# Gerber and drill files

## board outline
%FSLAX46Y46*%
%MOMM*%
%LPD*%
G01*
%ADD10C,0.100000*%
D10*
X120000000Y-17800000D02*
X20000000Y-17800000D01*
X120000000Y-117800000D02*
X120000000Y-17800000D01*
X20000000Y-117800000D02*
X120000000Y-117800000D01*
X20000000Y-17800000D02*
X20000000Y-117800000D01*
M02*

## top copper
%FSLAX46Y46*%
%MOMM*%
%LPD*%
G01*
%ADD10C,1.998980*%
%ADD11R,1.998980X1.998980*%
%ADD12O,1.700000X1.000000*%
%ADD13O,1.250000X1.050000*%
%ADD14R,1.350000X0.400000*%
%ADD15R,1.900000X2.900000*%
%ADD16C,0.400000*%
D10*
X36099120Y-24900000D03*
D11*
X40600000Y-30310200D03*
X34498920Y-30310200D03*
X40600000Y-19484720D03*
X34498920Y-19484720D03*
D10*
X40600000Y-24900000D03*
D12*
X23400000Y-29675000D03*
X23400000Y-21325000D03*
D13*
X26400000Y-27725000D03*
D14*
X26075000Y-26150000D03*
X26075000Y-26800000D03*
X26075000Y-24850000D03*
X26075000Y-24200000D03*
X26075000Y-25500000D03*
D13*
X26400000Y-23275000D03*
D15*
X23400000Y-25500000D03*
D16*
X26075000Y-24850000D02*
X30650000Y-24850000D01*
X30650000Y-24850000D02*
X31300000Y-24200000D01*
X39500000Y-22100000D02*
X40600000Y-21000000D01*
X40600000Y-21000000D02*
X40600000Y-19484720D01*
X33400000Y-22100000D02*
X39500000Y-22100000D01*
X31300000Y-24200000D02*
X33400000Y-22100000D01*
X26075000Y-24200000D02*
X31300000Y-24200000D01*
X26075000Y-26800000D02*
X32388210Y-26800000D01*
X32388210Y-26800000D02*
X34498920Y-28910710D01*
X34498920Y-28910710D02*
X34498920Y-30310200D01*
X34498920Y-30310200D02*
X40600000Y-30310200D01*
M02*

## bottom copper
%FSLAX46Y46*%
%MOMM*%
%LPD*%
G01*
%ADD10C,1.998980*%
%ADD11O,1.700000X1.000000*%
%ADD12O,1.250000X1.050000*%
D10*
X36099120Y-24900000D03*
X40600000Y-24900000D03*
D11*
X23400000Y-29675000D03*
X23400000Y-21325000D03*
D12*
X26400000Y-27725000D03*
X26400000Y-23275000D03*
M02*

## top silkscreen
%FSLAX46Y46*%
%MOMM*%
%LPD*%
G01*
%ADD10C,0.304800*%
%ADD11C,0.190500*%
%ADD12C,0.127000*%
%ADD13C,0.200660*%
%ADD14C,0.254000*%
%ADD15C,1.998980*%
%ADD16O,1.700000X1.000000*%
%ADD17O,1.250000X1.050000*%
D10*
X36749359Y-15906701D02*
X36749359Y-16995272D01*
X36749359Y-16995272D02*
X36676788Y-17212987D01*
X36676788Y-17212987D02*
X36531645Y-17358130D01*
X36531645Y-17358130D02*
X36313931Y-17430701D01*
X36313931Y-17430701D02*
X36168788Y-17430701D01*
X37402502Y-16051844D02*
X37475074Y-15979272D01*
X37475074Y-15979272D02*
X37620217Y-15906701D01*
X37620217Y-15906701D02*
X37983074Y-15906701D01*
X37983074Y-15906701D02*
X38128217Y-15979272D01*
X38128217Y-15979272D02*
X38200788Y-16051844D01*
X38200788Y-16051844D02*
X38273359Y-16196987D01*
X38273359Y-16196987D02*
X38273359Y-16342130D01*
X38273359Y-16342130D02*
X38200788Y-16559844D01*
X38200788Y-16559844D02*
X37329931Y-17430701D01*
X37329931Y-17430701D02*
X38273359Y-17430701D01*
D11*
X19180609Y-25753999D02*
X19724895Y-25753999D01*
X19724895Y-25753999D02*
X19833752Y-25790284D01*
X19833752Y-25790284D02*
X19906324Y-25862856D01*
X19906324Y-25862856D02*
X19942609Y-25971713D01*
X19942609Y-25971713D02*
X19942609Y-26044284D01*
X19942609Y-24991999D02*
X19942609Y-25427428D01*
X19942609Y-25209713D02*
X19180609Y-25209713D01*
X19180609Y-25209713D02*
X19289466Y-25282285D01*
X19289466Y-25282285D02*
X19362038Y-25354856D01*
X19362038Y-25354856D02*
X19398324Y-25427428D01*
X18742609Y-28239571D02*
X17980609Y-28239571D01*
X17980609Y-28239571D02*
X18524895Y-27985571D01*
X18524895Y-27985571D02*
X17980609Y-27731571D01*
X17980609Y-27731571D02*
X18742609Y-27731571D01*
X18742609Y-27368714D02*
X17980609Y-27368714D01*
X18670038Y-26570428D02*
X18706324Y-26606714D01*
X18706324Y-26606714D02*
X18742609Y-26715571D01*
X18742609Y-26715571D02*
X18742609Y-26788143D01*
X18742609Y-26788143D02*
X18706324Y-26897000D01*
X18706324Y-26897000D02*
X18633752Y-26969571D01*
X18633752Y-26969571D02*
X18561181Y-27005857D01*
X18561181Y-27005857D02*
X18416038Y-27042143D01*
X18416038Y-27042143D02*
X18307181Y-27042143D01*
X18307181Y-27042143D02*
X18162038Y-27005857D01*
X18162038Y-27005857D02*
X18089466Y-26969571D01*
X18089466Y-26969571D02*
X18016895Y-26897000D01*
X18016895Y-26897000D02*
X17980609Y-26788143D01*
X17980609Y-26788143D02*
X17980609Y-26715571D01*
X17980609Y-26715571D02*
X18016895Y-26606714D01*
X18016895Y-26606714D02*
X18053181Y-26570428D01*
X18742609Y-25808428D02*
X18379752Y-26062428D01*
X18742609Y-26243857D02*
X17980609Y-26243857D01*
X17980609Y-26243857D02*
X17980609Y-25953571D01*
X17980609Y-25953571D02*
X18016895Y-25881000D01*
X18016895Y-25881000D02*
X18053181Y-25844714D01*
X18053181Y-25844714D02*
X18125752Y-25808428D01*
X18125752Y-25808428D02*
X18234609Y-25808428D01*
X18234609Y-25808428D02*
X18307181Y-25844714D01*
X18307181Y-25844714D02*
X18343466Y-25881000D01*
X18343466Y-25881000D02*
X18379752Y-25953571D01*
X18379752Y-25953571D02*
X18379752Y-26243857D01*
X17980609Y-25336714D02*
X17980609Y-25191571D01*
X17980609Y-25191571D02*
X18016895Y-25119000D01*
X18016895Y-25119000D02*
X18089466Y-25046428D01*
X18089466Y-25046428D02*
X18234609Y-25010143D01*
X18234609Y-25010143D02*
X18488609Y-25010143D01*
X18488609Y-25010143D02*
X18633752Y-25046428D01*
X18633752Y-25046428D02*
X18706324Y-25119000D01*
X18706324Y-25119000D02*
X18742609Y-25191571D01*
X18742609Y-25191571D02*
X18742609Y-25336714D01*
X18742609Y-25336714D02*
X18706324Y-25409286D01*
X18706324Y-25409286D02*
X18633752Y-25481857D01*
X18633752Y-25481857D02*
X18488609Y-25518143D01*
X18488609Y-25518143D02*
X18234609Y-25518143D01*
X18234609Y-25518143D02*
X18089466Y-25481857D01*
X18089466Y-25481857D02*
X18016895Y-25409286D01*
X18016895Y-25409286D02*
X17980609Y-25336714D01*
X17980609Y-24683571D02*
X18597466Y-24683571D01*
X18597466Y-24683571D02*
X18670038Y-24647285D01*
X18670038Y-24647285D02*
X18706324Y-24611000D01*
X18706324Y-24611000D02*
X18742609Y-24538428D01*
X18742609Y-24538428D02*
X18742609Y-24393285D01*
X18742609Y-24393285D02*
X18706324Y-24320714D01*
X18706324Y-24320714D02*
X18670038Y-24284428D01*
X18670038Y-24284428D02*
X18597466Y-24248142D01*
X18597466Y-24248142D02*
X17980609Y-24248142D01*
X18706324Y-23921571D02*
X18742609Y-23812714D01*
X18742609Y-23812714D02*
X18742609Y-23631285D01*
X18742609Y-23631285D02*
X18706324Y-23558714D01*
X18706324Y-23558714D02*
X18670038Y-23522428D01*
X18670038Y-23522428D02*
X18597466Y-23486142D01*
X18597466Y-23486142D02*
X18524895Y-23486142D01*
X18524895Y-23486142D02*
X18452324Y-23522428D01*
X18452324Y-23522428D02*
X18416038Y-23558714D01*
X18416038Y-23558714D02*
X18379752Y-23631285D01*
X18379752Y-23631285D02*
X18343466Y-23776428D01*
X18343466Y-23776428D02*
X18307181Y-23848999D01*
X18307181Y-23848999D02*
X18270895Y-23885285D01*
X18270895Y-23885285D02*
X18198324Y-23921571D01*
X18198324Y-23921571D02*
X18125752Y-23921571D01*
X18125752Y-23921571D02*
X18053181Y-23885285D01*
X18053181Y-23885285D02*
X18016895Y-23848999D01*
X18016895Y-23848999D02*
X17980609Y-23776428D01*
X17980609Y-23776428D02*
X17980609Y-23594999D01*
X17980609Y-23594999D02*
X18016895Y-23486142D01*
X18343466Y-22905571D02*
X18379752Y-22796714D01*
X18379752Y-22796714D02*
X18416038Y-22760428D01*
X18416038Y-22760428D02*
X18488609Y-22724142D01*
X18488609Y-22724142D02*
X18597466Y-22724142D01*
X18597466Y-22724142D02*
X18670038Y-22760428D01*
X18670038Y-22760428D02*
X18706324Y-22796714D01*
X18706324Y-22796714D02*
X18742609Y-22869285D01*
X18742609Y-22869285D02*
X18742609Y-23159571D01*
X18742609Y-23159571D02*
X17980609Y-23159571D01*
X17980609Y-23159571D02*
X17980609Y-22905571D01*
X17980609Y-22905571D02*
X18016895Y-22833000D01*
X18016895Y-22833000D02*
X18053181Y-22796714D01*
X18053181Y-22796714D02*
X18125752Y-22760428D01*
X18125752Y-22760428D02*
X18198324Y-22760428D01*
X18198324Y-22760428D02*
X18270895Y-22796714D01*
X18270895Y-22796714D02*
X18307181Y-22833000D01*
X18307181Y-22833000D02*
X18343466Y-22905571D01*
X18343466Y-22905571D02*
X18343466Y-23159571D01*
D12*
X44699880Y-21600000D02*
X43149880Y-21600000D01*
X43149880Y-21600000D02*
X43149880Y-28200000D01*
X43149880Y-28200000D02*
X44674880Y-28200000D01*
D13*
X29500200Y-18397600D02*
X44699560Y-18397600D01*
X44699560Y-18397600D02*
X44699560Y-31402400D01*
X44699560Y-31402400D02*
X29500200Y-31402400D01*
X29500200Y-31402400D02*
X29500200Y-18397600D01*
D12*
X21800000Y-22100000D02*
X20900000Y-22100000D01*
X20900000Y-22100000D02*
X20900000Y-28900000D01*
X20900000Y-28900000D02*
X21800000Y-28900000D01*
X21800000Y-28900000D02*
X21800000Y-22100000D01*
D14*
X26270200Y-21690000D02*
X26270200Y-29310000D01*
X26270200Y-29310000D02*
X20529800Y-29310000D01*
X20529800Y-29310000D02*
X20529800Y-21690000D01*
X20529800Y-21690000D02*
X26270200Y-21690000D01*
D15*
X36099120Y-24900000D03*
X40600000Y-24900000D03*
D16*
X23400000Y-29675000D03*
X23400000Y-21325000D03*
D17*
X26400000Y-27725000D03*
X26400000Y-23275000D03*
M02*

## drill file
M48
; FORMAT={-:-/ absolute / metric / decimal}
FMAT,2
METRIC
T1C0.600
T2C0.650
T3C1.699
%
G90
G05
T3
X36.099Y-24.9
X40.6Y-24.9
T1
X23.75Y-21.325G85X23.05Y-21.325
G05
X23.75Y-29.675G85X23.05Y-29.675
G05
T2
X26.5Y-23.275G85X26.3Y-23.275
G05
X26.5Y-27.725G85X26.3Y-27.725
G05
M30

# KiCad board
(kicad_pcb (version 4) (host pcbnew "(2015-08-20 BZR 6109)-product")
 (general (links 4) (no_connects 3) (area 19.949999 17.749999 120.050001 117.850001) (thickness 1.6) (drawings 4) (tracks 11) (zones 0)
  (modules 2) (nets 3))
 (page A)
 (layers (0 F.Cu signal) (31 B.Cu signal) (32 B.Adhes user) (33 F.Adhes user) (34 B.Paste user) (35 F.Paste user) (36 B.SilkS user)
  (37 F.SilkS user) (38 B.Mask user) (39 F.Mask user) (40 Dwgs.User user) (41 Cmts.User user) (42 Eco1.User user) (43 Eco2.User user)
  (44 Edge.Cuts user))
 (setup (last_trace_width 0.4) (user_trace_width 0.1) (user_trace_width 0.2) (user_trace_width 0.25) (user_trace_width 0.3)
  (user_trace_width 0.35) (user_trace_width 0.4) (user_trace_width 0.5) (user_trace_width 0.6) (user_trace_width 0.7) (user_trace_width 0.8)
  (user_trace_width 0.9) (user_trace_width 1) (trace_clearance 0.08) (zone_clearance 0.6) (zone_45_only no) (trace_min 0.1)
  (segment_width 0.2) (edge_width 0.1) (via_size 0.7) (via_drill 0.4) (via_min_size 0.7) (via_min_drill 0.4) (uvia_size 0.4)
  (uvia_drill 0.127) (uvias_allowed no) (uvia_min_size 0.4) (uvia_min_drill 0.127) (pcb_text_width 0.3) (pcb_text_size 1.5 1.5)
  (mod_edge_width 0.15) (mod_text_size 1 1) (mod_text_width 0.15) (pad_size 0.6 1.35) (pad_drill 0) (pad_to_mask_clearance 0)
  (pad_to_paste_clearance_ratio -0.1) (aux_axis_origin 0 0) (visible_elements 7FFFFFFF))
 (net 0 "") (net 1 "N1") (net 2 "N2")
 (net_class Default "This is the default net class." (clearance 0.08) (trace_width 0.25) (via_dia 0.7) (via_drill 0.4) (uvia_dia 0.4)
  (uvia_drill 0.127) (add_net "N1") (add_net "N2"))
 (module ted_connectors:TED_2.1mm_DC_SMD (layer F.Cu) (at 37.09988 24.9)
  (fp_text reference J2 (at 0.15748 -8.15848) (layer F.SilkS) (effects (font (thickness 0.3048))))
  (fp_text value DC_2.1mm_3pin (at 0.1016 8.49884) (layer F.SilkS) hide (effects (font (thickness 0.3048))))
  (fp_line (start 7.6 -3.3) (end 6.05 -3.3) (layer F.SilkS) (width 0.127))
  (fp_line (start 6.05 -3.3) (end 6.05 3.3) (layer F.SilkS) (width 0.127))
  (fp_line (start 6.05 3.3) (end 7.575 3.3) (layer F.SilkS) (width 0.127))
  (fp_line (start -7.59968 -6.5024) (end 7.59968 -6.5024) (layer F.SilkS) (width 0.20066))
  (fp_line (start 7.59968 -6.5024) (end 7.59968 6.5024) (layer F.SilkS) (width 0.20066))
  (fp_line (start 7.59968 6.5024) (end -7.59968 6.5024) (layer F.SilkS) (width 0.20066))
  (fp_line (start -7.59968 6.5024) (end -7.59968 -6.5024) (layer F.SilkS) (width 0.20066))
  (pad "" np_thru_hole circle (at -1.00076 0) (size 1.99898 1.99898) (drill 1.69926) (layers *.Cu *.Mask F.SilkS))
  (pad 1 smd rect (at 3.50012 5.4102) (size 1.99898 1.99898) (layers F.Cu F.Paste F.Mask) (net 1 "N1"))
  (pad 1 smd rect (at -2.60096 5.4102) (size 1.99898 1.99898) (layers F.Cu F.Paste F.Mask) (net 1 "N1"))
  (pad 2 smd rect (at 3.50012 -5.41528) (size 1.99898 1.99898) (layers F.Cu F.Paste F.Mask) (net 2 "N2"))
  (pad 3 smd rect (at -2.60096 -5.41528) (size 1.99898 1.99898) (layers F.Cu F.Paste F.Mask))
  (pad "" np_thru_hole circle (at 3.50012 0) (size 1.99898 1.99898) (drill 1.69926) (layers *.Cu *.Mask F.SilkS)))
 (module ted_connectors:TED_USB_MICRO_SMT (layer F.Cu) (at 23.4 25.5 270)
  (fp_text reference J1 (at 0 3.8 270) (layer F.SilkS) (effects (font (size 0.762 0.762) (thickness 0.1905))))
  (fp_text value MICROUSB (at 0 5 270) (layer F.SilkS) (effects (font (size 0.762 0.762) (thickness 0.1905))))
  (fp_line (start -3.4 1.6) (end -3.4 2.5) (layer F.SilkS) (width 0.127))
  (fp_line (start -3.4 2.5) (end 3.4 2.5) (layer F.SilkS) (width 0.127))
  (fp_line (start 3.4 2.5) (end 3.4 1.6) (layer F.SilkS) (width 0.127))
  (fp_line (start 3.4 1.6) (end -3.4 1.6) (layer F.SilkS) (width 0.127))
  (fp_line (start -3.81 -2.8702) (end 3.81 -2.8702) (layer F.SilkS) (width 0.254))
  (fp_line (start 3.81 -2.8702) (end 3.81 2.8702) (layer F.SilkS) (width 0.254))
  (fp_line (start 3.81 2.8702) (end -3.81 2.8702) (layer F.SilkS) (width 0.254))
  (fp_line (start -3.81 2.8702) (end -3.81 -2.8702) (layer F.SilkS) (width 0.254))
  (pad "" np_thru_hole oval (at 4.175 0 270) (size 1 1.7) (drill oval 0.6 1.3) (layers *.Cu *.Mask F.SilkS) (clearance 0.127))
  (pad "" np_thru_hole oval (at -4.175 0 270) (size 1 1.7) (drill oval 0.6 1.3) (layers *.Cu *.Mask F.SilkS) (clearance 0.127))
  (pad "" np_thru_hole oval (at 2.225 -3 270) (size 1.05 1.25) (drill oval 0.65 0.85) (layers *.Cu *.Mask F.SilkS) (clearance 0.127))
  (pad 2 smd rect (at 0.65 -2.675 270) (size 0.4 1.35) (layers F.Cu F.Paste F.Mask) (clearance 0.127))
  (pad 1 smd rect (at 1.3 -2.675 270) (size 0.4 1.35) (layers F.Cu F.Paste F.Mask) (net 1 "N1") (clearance 0.127))
  (pad 4 smd rect (at -0.65 -2.675 270) (size 0.4 1.35) (layers F.Cu F.Paste F.Mask) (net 2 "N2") (clearance 0.127))
  (pad 5 smd rect (at -1.3 -2.675 270) (size 0.4 1.35) (layers F.Cu F.Paste F.Mask) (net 2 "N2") (clearance 0.127))
  (pad 3 smd rect (at 0 -2.675 270) (size 0.4 1.35) (layers F.Cu F.Paste F.Mask) (clearance 0.127))
  (pad "" np_thru_hole oval (at -2.225 -3 270) (size 1.05 1.25) (drill oval 0.65 0.85) (layers *.Cu *.Mask F.SilkS) (clearance 0.127))
  (pad PAD smd rect (at 0 0 270) (size 2.9 1.9) (layers F.Cu F.Paste F.Mask)))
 (gr_line (start 120 17.8) (end 20 17.8) (angle 90) (layer Edge.Cuts) (width 0.1))
 (gr_line (start 120 117.8) (end 120 17.8) (angle 90) (layer Edge.Cuts) (width 0.1))
 (gr_line (start 20 117.8) (end 120 117.8) (angle 90) (layer Edge.Cuts) (width 0.1))
 (gr_line (start 20 17.8) (end 20 117.8) (angle 90) (layer Edge.Cuts) (width 0.1))
 (segment (start 26.075 24.85) (end 30.65 24.85) (width 0.4) (layer F.Cu) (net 2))
 (segment (start 30.65 24.85) (end 31.3 24.2) (width 0.4) (layer F.Cu) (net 2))
 (segment (start 39.5 22.1) (end 40.6 21) (width 0.4) (layer F.Cu) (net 2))
 (segment (start 40.6 21) (end 40.6 19.48472) (width 0.4) (layer F.Cu) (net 2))
 (segment (start 33.4 22.1) (end 39.5 22.1) (width 0.4) (layer F.Cu) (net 2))
 (segment (start 31.3 24.2) (end 33.4 22.1) (width 0.4) (layer F.Cu) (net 2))
 (segment (start 26.075 24.2) (end 31.3 24.2) (width 0.4) (layer F.Cu) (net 2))
 (segment (start 26.075 26.8) (end 32.38821 26.8) (width 0.4) (layer F.Cu) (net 1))
 (segment (start 32.38821 26.8) (end 34.49892 28.91071) (width 0.4) (layer F.Cu) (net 1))
 (segment (start 34.49892 28.91071) (end 34.49892 30.3102) (width 0.4) (layer F.Cu) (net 1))
 (segment (start 34.49892 30.3102) (end 40.6 30.3102) (width 0.4) (layer F.Cu) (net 1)))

